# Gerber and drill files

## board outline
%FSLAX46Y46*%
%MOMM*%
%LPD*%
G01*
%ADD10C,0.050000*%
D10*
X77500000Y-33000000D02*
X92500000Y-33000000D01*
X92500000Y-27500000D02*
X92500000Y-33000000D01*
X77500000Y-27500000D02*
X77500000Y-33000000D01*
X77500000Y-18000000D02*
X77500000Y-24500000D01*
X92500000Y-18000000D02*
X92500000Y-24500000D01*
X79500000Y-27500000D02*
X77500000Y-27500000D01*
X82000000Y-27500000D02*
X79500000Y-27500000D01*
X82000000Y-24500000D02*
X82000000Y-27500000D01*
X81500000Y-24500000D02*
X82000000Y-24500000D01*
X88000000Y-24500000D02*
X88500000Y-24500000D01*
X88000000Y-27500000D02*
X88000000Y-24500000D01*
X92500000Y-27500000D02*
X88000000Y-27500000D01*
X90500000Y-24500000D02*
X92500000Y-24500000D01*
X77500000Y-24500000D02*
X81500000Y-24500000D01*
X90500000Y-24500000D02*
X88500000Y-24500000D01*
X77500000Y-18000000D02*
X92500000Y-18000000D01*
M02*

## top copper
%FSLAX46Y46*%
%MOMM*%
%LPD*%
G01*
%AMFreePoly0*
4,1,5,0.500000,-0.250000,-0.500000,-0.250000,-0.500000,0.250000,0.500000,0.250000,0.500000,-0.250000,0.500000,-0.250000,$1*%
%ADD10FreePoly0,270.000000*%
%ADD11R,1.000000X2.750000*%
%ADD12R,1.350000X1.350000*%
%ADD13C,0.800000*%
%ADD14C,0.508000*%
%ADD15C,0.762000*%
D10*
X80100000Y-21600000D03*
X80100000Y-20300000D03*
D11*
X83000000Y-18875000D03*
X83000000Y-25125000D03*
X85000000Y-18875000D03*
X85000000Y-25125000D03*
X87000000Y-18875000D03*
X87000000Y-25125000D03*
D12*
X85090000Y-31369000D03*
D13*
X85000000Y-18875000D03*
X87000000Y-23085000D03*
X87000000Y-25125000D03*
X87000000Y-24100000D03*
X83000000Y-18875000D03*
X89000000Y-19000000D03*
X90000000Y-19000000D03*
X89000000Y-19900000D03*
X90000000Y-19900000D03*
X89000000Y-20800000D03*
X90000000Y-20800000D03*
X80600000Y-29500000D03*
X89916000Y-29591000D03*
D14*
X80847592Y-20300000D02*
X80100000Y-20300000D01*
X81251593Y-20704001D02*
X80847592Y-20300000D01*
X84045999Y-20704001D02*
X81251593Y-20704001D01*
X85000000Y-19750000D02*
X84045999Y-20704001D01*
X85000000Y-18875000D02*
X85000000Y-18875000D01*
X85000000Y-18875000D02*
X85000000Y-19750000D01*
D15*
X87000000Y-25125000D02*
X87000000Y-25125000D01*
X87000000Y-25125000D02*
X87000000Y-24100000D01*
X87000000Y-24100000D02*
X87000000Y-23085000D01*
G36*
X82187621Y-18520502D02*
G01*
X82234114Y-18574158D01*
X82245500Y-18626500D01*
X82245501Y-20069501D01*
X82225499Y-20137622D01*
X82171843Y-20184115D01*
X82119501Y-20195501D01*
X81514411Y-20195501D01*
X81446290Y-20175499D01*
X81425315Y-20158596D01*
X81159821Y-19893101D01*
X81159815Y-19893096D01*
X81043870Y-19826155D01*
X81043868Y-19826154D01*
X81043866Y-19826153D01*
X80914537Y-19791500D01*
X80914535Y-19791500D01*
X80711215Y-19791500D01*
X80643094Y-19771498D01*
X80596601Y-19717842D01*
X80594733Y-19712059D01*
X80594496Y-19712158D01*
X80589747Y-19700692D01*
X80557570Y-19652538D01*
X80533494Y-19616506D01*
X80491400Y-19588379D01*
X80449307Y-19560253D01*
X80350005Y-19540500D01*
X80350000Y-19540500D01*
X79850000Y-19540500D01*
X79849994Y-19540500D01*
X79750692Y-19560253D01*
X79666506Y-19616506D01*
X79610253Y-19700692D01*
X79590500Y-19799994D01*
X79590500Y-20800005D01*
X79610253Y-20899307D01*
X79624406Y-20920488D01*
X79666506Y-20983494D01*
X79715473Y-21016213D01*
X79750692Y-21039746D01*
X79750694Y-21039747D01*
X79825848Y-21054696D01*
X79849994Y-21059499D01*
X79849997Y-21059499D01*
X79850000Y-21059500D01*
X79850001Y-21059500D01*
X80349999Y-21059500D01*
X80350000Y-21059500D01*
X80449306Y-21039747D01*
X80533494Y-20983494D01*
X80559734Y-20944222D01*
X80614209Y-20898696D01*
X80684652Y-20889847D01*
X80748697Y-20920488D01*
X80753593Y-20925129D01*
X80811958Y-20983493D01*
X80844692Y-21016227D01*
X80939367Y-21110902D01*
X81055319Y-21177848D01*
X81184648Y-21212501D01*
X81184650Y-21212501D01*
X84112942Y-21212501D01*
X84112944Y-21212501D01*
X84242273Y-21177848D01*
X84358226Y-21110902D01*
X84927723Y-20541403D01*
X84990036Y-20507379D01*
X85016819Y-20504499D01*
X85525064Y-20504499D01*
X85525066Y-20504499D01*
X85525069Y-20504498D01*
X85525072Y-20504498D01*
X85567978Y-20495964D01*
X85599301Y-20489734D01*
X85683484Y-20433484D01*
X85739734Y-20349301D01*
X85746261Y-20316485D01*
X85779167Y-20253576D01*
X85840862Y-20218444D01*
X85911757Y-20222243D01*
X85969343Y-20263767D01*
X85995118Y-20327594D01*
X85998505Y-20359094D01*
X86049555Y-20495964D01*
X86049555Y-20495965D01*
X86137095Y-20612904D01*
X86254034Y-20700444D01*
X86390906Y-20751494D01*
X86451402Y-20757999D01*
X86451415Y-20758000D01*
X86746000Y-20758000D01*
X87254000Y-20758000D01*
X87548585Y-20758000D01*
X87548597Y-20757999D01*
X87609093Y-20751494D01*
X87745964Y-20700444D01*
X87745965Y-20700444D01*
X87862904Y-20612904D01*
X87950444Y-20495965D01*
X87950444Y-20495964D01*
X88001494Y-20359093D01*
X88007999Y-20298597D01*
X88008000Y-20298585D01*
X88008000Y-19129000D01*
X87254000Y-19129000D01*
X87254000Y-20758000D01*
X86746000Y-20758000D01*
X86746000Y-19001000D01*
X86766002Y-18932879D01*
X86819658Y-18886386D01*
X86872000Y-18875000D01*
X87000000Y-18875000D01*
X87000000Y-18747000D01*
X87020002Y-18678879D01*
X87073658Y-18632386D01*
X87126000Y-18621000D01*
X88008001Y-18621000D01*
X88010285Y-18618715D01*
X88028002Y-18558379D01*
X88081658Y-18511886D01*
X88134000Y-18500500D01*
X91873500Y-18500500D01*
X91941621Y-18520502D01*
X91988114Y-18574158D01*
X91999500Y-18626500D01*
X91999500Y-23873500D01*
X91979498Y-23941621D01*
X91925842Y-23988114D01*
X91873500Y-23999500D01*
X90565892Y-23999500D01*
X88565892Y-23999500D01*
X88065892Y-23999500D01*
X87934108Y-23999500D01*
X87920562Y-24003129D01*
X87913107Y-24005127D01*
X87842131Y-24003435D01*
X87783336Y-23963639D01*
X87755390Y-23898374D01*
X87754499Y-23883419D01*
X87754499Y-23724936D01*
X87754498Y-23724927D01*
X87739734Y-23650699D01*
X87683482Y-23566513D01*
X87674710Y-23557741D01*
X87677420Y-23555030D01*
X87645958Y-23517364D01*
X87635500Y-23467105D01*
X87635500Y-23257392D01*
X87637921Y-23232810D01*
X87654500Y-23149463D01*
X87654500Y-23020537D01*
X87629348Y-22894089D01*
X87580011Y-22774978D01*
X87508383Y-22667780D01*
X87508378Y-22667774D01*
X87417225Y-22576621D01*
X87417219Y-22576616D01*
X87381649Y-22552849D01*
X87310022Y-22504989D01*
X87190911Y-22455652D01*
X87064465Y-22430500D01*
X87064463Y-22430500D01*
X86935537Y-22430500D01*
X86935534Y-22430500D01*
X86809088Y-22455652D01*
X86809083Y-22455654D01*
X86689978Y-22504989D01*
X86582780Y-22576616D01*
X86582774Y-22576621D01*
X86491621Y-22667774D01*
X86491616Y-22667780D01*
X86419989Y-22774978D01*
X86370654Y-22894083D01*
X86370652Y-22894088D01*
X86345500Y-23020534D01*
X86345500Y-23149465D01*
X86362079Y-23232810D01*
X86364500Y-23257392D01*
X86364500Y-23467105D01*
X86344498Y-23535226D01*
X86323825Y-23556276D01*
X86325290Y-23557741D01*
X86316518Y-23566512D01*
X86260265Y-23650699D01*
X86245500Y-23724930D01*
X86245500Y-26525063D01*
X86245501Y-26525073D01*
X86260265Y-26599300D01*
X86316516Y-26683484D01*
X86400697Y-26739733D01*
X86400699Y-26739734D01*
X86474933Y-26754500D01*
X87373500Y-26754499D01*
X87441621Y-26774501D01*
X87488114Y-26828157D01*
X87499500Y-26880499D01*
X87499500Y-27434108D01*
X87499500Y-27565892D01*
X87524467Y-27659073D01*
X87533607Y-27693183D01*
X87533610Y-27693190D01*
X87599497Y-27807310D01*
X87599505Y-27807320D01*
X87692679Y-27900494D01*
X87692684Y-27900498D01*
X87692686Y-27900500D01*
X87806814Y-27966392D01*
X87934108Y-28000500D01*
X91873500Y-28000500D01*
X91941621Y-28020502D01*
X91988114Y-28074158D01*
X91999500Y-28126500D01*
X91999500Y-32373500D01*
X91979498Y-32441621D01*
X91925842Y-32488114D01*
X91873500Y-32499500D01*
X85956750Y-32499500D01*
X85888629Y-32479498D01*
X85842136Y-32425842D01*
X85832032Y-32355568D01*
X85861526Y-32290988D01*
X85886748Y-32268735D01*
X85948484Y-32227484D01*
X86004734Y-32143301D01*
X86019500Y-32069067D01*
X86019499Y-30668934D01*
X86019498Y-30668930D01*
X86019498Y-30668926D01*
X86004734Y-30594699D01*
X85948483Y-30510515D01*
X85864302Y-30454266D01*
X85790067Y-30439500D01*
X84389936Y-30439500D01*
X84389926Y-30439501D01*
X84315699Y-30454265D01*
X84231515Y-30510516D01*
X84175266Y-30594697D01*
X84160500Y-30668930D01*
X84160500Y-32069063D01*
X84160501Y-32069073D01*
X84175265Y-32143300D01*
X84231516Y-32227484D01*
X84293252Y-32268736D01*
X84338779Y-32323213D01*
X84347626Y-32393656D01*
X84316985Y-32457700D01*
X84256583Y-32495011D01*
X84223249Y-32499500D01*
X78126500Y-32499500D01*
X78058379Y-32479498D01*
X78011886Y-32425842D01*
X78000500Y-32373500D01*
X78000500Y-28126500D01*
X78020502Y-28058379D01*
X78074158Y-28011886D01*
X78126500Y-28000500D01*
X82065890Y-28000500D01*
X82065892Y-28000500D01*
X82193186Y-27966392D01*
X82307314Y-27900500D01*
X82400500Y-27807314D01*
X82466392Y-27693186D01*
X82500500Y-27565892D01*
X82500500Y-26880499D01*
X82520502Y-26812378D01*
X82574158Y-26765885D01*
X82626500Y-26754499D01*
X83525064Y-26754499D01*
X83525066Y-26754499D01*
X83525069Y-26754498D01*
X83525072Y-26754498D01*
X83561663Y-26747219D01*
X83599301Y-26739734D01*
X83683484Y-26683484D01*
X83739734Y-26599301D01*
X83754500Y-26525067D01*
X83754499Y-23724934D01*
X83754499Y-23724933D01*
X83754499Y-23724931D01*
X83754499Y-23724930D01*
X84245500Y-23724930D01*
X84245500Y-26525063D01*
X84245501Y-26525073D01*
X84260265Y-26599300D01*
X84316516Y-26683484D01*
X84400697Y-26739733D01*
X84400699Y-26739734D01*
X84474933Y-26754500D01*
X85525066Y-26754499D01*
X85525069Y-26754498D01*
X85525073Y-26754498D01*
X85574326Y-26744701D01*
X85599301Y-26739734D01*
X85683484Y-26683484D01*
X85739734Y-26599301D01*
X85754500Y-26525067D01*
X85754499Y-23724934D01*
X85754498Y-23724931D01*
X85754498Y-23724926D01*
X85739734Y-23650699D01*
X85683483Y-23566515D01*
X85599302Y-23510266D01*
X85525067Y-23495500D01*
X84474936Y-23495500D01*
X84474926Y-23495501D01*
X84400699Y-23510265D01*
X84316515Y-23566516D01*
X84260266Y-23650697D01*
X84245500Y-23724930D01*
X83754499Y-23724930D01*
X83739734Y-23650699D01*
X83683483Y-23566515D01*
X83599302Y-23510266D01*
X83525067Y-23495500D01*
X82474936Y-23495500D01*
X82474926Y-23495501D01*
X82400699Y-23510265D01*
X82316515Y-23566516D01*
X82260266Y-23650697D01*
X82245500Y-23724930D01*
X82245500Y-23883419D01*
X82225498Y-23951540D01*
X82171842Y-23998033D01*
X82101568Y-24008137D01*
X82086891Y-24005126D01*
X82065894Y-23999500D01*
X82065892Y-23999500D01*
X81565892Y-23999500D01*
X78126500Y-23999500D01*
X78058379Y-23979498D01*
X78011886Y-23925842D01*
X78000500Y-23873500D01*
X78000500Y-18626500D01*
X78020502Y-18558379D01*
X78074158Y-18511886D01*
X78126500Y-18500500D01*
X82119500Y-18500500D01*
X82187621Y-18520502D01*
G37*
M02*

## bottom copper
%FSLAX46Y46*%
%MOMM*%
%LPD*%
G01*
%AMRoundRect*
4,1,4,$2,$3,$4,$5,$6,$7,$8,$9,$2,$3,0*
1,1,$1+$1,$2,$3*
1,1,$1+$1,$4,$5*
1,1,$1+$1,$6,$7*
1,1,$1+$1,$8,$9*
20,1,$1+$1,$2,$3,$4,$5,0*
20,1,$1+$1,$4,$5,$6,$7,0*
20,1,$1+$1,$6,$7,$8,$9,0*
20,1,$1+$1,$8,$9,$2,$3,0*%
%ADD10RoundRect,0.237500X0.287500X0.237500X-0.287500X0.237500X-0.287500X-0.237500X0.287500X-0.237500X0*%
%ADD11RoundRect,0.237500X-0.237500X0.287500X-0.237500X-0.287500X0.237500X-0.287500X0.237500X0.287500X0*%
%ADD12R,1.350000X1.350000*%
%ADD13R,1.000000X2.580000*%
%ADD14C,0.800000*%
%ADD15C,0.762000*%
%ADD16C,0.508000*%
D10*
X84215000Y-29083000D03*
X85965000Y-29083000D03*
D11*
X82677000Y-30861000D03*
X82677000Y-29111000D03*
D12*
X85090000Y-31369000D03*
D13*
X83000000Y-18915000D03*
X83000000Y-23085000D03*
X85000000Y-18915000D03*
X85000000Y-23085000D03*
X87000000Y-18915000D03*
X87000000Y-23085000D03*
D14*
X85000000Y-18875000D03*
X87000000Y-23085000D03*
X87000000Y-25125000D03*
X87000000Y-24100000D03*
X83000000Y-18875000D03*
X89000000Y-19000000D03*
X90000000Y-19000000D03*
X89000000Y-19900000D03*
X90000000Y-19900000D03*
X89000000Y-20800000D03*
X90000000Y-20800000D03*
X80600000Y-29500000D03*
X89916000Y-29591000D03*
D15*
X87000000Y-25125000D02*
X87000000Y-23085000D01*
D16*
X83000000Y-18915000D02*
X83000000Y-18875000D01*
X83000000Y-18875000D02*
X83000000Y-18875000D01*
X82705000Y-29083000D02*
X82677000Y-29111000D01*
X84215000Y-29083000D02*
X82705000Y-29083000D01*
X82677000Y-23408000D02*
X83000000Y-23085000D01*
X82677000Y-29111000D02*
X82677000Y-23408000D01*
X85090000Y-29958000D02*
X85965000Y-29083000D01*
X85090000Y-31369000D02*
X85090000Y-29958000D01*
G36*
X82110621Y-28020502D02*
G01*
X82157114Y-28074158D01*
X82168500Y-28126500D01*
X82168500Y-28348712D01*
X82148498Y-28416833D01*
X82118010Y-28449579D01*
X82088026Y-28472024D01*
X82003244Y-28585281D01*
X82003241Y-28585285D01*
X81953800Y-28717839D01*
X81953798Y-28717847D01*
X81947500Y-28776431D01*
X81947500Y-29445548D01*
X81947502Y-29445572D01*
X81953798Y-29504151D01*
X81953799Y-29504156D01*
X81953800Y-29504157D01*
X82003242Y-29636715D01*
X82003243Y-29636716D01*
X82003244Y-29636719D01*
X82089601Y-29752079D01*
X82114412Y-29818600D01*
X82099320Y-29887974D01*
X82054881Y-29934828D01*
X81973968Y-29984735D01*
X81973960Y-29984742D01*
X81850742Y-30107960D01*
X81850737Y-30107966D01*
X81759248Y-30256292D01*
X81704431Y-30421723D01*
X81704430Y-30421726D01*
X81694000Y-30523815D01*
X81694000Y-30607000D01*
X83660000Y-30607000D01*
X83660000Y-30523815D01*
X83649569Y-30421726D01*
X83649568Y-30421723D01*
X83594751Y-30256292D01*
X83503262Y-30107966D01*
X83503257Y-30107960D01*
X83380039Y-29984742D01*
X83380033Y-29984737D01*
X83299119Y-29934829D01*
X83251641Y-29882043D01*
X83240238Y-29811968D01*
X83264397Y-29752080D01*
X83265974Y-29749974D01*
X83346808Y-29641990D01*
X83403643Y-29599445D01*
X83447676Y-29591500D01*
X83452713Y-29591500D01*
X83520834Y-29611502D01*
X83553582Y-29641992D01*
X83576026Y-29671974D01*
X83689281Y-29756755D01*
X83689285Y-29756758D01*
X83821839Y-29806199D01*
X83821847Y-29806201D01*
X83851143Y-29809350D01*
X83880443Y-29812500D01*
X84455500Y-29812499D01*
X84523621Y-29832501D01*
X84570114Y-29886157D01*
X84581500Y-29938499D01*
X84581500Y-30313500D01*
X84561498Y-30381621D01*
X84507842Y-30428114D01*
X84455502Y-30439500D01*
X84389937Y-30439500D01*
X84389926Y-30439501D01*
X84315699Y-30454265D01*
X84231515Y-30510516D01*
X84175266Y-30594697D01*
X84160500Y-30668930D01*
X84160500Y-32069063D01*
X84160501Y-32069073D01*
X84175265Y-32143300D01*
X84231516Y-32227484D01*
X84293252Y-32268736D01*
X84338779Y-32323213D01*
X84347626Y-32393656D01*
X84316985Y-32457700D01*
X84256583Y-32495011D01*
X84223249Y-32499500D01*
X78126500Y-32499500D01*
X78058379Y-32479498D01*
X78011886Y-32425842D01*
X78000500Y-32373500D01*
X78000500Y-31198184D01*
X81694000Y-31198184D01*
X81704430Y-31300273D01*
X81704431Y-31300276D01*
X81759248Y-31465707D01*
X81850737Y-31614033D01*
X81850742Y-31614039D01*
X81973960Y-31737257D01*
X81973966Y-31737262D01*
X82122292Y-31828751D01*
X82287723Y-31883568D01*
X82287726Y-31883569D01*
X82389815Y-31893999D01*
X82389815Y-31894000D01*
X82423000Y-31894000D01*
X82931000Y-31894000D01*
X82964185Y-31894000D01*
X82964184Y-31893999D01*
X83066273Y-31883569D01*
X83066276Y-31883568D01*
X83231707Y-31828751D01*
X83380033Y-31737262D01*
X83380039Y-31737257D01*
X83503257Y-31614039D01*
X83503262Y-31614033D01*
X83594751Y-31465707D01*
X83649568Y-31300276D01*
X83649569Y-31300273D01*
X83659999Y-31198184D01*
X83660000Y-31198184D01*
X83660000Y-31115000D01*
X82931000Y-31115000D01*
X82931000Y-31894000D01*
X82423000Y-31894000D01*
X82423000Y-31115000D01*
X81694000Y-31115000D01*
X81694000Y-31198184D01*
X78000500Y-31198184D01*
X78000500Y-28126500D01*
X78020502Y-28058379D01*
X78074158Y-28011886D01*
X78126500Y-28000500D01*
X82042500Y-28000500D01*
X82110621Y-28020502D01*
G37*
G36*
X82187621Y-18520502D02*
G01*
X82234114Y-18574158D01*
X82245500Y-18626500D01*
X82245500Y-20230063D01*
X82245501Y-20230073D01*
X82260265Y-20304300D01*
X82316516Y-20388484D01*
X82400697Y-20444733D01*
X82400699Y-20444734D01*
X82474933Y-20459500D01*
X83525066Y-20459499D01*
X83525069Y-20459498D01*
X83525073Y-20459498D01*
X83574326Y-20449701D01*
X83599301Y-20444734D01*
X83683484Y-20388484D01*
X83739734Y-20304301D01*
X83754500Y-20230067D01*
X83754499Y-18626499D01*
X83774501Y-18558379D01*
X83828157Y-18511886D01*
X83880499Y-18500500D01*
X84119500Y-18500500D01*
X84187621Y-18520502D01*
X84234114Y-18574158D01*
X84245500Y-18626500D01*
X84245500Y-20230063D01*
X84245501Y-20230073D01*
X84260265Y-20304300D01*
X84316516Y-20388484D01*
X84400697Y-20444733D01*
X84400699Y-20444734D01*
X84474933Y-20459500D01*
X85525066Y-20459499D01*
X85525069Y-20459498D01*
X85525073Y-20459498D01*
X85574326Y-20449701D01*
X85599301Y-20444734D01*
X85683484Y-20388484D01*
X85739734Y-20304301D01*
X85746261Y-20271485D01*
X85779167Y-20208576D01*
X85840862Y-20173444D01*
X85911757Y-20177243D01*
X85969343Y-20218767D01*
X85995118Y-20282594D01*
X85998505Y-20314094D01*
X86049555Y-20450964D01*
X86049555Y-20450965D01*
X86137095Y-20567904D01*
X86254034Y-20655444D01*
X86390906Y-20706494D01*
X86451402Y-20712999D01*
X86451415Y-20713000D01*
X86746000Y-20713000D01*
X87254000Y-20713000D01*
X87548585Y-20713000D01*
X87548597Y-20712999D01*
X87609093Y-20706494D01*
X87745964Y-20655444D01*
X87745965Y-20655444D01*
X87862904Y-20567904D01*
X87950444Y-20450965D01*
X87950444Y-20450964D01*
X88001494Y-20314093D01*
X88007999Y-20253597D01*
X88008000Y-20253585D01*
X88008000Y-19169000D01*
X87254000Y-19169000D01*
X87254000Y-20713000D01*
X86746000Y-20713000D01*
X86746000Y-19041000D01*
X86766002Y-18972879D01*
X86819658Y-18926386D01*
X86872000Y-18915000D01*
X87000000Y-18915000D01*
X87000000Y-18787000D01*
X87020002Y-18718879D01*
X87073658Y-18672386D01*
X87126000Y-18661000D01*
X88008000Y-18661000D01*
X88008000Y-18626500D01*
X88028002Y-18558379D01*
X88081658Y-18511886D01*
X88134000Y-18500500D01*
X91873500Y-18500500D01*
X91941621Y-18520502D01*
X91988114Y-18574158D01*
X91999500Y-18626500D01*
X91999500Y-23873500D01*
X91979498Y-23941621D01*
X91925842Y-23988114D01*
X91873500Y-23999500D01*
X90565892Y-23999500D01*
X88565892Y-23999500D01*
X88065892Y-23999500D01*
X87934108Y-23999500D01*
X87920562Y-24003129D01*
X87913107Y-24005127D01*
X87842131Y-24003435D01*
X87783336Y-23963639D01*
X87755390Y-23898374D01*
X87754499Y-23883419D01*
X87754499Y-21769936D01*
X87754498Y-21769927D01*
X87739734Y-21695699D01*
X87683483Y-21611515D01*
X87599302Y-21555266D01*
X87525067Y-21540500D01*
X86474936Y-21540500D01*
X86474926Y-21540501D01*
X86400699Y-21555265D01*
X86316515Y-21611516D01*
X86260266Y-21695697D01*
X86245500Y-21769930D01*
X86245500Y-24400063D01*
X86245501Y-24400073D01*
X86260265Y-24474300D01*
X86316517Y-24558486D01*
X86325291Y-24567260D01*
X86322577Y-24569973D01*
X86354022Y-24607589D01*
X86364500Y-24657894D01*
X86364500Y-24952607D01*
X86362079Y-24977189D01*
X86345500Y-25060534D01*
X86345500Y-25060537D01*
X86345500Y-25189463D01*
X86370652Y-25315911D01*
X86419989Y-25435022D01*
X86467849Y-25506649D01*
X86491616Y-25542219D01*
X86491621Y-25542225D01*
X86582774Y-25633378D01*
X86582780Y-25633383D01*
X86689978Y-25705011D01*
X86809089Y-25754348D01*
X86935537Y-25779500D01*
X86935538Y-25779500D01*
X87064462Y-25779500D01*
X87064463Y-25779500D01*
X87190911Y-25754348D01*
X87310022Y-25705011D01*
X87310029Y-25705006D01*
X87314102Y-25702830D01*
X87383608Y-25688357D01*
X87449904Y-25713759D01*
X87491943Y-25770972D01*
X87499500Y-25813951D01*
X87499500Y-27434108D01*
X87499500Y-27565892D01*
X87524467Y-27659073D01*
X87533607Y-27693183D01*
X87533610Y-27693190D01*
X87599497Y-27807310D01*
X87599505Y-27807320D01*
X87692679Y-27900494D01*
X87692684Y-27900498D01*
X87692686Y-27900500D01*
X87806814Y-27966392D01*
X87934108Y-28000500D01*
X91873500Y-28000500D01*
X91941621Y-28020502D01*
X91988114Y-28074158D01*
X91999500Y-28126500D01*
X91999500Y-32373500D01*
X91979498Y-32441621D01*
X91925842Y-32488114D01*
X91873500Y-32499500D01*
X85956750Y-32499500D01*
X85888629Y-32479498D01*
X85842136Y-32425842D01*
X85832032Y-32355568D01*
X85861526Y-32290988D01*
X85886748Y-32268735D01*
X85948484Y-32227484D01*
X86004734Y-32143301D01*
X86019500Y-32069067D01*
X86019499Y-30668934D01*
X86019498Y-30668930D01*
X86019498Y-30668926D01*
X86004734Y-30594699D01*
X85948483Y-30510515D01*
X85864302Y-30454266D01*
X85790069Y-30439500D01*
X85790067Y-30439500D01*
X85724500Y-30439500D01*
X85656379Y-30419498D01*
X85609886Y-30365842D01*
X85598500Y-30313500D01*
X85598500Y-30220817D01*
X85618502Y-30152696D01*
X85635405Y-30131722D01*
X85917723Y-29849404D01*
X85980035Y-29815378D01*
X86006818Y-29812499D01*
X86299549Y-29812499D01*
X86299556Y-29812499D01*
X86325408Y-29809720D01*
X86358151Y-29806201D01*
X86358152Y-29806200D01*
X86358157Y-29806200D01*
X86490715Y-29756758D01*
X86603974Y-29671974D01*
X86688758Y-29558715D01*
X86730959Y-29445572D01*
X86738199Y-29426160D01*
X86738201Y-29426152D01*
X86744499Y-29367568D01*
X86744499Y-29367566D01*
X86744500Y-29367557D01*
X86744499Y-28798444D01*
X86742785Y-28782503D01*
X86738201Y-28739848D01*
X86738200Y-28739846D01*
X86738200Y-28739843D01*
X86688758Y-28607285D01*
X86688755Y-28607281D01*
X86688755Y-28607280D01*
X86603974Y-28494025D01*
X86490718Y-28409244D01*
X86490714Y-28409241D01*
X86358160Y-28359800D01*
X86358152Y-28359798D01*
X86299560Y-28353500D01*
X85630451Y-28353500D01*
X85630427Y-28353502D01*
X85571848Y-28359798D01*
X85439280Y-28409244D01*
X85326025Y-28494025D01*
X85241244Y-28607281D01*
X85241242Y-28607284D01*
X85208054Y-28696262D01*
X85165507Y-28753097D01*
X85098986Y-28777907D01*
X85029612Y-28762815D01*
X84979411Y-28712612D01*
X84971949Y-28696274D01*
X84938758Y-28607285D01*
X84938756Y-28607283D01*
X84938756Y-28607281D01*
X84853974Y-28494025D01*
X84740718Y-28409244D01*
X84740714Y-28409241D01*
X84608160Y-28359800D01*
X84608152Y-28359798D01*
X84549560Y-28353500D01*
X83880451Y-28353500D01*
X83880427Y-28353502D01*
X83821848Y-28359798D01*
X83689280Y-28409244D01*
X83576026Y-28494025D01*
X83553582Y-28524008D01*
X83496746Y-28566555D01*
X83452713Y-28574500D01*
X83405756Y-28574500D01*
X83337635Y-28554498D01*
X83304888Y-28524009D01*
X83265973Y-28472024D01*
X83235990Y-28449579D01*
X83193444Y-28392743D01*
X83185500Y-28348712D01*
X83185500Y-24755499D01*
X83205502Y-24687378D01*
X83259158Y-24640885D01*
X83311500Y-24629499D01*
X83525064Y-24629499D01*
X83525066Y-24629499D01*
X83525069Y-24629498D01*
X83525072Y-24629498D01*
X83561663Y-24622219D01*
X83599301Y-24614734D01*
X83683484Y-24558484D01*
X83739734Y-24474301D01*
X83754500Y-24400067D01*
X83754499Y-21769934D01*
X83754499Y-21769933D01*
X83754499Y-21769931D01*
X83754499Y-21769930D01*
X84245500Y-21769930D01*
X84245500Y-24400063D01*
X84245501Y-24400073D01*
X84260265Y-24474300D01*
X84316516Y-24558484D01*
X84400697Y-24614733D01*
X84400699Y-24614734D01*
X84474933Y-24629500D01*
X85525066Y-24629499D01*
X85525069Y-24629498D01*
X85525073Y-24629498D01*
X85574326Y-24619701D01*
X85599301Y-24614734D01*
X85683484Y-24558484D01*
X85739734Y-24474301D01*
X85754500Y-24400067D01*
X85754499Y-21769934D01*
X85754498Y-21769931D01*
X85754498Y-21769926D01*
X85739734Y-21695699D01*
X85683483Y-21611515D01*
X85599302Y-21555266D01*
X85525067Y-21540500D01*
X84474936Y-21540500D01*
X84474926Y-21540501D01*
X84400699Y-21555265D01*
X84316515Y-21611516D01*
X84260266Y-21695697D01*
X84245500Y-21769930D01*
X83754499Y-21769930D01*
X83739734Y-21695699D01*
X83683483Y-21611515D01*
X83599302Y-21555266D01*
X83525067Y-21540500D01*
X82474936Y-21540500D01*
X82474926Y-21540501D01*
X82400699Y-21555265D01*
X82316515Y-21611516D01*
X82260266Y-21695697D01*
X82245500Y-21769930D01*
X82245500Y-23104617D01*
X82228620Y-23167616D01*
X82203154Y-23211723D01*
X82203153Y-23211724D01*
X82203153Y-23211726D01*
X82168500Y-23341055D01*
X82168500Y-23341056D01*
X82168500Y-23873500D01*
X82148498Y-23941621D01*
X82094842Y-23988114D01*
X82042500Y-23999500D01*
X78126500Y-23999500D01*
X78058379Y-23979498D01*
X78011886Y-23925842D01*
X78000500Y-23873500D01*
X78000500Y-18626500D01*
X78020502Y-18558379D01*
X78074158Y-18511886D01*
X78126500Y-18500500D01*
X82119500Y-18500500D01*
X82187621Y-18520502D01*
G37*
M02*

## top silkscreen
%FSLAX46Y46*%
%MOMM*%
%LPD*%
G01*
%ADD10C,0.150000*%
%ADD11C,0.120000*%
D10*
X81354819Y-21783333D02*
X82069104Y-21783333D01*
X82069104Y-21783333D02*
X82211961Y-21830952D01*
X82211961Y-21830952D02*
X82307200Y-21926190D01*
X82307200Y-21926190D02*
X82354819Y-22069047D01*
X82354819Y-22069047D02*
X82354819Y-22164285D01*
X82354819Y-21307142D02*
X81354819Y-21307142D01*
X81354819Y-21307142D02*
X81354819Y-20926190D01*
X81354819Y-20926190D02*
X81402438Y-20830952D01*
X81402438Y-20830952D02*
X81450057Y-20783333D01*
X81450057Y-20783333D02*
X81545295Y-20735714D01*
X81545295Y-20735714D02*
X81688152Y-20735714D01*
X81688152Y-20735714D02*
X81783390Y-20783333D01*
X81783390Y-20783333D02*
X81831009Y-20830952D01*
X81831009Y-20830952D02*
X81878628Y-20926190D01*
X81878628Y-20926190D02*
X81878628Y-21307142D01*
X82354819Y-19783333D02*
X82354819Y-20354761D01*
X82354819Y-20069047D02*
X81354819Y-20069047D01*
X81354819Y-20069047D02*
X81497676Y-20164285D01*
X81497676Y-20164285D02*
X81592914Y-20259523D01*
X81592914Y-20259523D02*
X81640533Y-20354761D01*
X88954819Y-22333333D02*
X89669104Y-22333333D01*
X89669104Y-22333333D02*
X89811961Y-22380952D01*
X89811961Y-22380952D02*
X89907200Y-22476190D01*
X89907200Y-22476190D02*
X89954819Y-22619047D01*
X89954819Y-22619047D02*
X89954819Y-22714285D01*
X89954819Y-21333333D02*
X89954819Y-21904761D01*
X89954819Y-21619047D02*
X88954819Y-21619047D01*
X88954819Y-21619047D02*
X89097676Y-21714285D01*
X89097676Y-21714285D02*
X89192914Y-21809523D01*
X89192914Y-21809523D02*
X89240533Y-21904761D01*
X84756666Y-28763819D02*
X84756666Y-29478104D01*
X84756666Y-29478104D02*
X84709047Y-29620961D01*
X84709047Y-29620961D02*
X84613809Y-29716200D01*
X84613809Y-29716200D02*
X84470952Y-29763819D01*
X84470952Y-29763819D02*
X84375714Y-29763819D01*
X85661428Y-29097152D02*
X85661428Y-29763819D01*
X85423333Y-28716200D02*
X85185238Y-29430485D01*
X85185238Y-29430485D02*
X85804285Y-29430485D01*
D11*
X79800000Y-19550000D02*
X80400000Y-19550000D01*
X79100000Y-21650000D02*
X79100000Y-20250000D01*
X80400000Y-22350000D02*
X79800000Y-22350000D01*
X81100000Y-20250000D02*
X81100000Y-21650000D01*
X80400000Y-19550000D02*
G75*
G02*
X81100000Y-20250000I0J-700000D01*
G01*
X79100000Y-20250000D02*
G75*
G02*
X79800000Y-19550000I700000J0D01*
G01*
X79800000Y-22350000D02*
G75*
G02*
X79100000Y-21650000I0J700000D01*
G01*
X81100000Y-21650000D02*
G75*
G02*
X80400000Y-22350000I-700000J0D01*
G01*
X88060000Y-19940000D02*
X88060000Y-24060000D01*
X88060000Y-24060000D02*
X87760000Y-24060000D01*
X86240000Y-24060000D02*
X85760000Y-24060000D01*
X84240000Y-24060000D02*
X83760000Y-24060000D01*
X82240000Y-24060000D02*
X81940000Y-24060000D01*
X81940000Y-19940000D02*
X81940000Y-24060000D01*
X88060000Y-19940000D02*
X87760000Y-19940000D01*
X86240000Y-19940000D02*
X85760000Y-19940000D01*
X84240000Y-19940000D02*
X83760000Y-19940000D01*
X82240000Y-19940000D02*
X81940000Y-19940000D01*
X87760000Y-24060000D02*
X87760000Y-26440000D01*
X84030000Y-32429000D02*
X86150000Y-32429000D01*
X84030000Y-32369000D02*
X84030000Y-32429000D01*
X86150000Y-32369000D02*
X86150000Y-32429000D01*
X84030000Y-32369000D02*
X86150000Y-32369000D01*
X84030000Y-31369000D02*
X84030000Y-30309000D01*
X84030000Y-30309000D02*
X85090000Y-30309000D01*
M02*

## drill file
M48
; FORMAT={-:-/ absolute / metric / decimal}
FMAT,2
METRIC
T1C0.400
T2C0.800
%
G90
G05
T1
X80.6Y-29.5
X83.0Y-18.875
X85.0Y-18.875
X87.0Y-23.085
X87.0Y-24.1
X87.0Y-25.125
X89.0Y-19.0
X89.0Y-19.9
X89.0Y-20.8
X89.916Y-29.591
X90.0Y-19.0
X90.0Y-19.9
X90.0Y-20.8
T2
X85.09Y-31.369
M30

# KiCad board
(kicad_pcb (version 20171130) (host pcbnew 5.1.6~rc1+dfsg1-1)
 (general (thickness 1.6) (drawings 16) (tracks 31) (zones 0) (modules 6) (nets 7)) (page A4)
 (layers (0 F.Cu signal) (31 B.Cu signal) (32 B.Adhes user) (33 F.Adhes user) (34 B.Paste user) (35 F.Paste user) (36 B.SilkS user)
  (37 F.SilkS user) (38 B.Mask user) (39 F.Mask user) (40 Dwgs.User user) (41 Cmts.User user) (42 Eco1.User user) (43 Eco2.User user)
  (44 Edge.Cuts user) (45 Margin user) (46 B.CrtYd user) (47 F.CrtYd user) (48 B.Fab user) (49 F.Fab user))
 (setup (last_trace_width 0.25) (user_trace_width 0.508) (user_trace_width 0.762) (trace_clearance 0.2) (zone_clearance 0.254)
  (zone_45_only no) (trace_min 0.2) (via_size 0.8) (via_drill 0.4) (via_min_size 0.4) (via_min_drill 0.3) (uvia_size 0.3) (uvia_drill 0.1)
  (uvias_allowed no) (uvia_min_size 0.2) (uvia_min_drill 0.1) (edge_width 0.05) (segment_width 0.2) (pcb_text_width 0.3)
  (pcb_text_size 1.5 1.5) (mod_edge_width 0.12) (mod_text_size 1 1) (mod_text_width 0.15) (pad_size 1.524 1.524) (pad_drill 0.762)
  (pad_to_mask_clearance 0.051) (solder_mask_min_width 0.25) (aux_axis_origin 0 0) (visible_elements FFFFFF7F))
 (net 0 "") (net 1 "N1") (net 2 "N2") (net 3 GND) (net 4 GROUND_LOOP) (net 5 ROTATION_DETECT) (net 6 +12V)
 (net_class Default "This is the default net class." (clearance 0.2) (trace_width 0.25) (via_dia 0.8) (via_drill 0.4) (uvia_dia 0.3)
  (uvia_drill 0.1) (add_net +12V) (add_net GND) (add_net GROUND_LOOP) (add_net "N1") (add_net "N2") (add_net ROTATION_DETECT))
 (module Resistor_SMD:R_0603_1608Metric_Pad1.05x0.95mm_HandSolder (layer B.Cu) (at 85.09 29.083 180)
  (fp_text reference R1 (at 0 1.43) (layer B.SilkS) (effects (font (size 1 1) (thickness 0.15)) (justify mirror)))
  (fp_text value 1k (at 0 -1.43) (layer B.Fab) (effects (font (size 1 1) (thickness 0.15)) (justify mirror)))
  (pad 2 smd roundrect (at 0.875 0 180) (size 1.05 0.95) (layers B.Cu B.Paste B.Mask) (roundrect_rratio 0.25) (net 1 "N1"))
  (pad 1 smd roundrect (at -0.875 0 180) (size 1.05 0.95) (layers B.Cu B.Paste B.Mask) (roundrect_rratio 0.25) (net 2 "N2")))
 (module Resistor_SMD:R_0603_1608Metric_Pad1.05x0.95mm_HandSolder (layer B.Cu) (at 82.677 29.986 270)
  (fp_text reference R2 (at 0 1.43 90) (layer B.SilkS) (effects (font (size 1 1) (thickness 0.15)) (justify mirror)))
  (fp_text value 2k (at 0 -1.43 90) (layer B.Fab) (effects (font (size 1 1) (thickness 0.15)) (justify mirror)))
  (pad 2 smd roundrect (at 0.875 0 270) (size 1.05 0.95) (layers B.Cu B.Paste B.Mask) (roundrect_rratio 0.25) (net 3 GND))
  (pad 1 smd roundrect (at -0.875 0 270) (size 1.05 0.95) (layers B.Cu B.Paste B.Mask) (roundrect_rratio 0.25) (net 1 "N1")))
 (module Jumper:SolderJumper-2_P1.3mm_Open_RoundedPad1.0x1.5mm (layer F.Cu) (at 80.1 20.95 270)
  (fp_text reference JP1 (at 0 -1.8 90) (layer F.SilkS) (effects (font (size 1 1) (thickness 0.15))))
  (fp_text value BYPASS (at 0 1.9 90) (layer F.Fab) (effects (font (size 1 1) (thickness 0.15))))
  (fp_line (start -1.4 0.3) (end -1.4 -0.3) (layer F.SilkS) (width 0.12))
  (fp_line (start 0.7 1) (end -0.7 1) (layer F.SilkS) (width 0.12))
  (fp_line (start 1.4 -0.3) (end 1.4 0.3) (layer F.SilkS) (width 0.12))
  (fp_line (start -0.7 -1) (end 0.7 -1) (layer F.SilkS) (width 0.12))
  (fp_arc (start -0.7 -0.3) (end -0.7 -1) (angle -90) (layer F.SilkS) (width 0.12))
  (fp_arc (start -0.7 0.3) (end -1.4 0.3) (angle -90) (layer F.SilkS) (width 0.12))
  (fp_arc (start 0.7 0.3) (end 0.7 1) (angle -90) (layer F.SilkS) (width 0.12))
  (fp_arc (start 0.7 -0.3) (end 1.4 -0.3) (angle -90) (layer F.SilkS) (width 0.12))
  (pad 2 smd custom (at 0.65 0 270) (size 1 0.5) (layers F.Cu F.Mask) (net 3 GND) (zone_connect 2)
   (options (clearance outline) (anchor rect)) (primitives))
  (pad 1 smd custom (at -0.65 0 270) (size 1 0.5) (layers F.Cu F.Mask) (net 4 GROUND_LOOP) (zone_connect 2)
   (options (clearance outline) (anchor rect)) (primitives)))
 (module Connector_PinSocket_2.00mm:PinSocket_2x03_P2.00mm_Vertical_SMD (layer F.Cu) (at 85 22 270)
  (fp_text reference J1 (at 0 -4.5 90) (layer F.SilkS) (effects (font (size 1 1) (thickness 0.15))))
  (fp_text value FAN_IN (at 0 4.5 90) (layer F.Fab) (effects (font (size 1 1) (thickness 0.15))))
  (fp_line (start -2.06 -3.06) (end 2.06 -3.06) (layer F.SilkS) (width 0.12))
  (fp_line (start 2.06 -3.06) (end 2.06 -2.76) (layer F.SilkS) (width 0.12))
  (fp_line (start 2.06 -1.24) (end 2.06 -0.76) (layer F.SilkS) (width 0.12))
  (fp_line (start 2.06 0.76) (end 2.06 1.24) (layer F.SilkS) (width 0.12))
  (fp_line (start 2.06 2.76) (end 2.06 3.06) (layer F.SilkS) (width 0.12))
  (fp_line (start -2.06 3.06) (end 2.06 3.06) (layer F.SilkS) (width 0.12))
  (fp_line (start -2.06 -3.06) (end -2.06 -2.76) (layer F.SilkS) (width 0.12))
  (fp_line (start -2.06 -1.24) (end -2.06 -0.76) (layer F.SilkS) (width 0.12))
  (fp_line (start -2.06 0.76) (end -2.06 1.24) (layer F.SilkS) (width 0.12))
  (fp_line (start -2.06 2.76) (end -2.06 3.06) (layer F.SilkS) (width 0.12))
  (fp_line (start 2.06 -2.76) (end 4.44 -2.76) (layer F.SilkS) (width 0.12))
  (pad 6 smd rect (at -3.125 2 270) (size 2.75 1) (layers F.Cu F.Paste F.Mask) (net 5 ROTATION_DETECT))
  (pad 5 smd rect (at 3.125 2 270) (size 2.75 1) (layers F.Cu F.Paste F.Mask))
  (pad 4 smd rect (at -3.125 0 270) (size 2.75 1) (layers F.Cu F.Paste F.Mask) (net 4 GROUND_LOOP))
  (pad 3 smd rect (at 3.125 0 270) (size 2.75 1) (layers F.Cu F.Paste F.Mask))
  (pad 2 smd rect (at -3.125 -2 270) (size 2.75 1) (layers F.Cu F.Paste F.Mask) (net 3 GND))
  (pad 1 smd rect (at 3.125 -2 270) (size 2.75 1) (layers F.Cu F.Paste F.Mask) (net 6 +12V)))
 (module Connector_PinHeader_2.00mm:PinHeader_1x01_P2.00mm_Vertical (layer F.Cu) (at 85.09 31.369)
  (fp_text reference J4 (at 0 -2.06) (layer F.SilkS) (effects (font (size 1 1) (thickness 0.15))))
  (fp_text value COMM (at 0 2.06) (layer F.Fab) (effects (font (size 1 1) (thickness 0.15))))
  (fp_line (start -1.06 1.06) (end 1.06 1.06) (layer F.SilkS) (width 0.12))
  (fp_line (start -1.06 1) (end -1.06 1.06) (layer F.SilkS) (width 0.12))
  (fp_line (start 1.06 1) (end 1.06 1.06) (layer F.SilkS) (width 0.12))
  (fp_line (start -1.06 1) (end 1.06 1) (layer F.SilkS) (width 0.12))
  (fp_line (start -1.06 0) (end -1.06 -1.06) (layer F.SilkS) (width 0.12))
  (fp_line (start -1.06 -1.06) (end 0 -1.06) (layer F.SilkS) (width 0.12))
  (pad 1 thru_hole rect (at 0 0) (size 1.35 1.35) (drill 0.8) (layers *.Cu *.Mask) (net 2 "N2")))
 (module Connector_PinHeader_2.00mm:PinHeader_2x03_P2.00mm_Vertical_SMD (layer B.Cu) (at 85 21 90)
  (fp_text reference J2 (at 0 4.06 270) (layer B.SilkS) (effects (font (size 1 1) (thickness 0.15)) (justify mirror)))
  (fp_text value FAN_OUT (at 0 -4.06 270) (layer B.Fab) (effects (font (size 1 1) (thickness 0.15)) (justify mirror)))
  (pad 6 smd rect (at 2.085 -2 90) (size 2.58 1) (layers B.Cu B.Paste B.Mask) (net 5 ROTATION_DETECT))
  (pad 5 smd rect (at -2.085 -2 90) (size 2.58 1) (layers B.Cu B.Paste B.Mask) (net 1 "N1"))
  (pad 4 smd rect (at 2.085 0 90) (size 2.58 1) (layers B.Cu B.Paste B.Mask) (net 4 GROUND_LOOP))
  (pad 3 smd rect (at -2.085 0 90) (size 2.58 1) (layers B.Cu B.Paste B.Mask))
  (pad 2 smd rect (at 2.085 2 90) (size 2.58 1) (layers B.Cu B.Paste B.Mask) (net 3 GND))
  (pad 1 smd rect (at -2.085 2 90) (size 2.58 1) (layers B.Cu B.Paste B.Mask) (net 6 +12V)))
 (gr_line (start 77.5 33) (end 92.5 33) (layer Edge.Cuts) (width 0.05))
 (gr_line (start 92.5 27.5) (end 92.5 33) (layer Edge.Cuts) (width 0.05))
 (gr_line (start 77.5 27.5) (end 77.5 33) (layer Edge.Cuts) (width 0.05))
 (gr_line (start 77.5 18) (end 77.5 24.5) (layer Edge.Cuts) (width 0.05))
 (gr_line (start 92.5 18) (end 92.5 24.5) (layer Edge.Cuts) (width 0.05))
 (gr_line (start 79.5 27.5) (end 77.5 27.5) (layer Edge.Cuts) (width 0.05))
 (gr_line (start 82 27.5) (end 79.5 27.5) (layer Edge.Cuts) (width 0.05))
 (gr_line (start 82 24.5) (end 82 27.5) (layer Edge.Cuts) (width 0.05))
 (gr_line (start 81.5 24.5) (end 82 24.5) (layer Edge.Cuts) (width 0.05))
 (gr_line (start 88 24.5) (end 88.5 24.5) (layer Edge.Cuts) (width 0.05))
 (gr_line (start 88 27.5) (end 88 24.5) (layer Edge.Cuts) (width 0.05))
 (gr_line (start 92.5 27.5) (end 88 27.5) (layer Edge.Cuts) (width 0.05))
 (gr_line (start 90.5 24.5) (end 92.5 24.5) (layer Edge.Cuts) (width 0.05))
 (gr_line (start 77.5 24.5) (end 81.5 24.5) (layer Edge.Cuts) (width 0.05))
 (gr_line (start 90.5 24.5) (end 88.5 24.5) (layer Edge.Cuts) (width 0.05))
 (gr_line (start 77.5 18) (end 92.5 18) (layer Edge.Cuts) (width 0.05))
 (segment (start 80.847592 20.3) (end 80.1 20.3) (width 0.508) (layer F.Cu) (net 4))
 (segment (start 81.251593 20.704001) (end 80.847592 20.3) (width 0.508) (layer F.Cu) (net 4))
 (segment (start 84.045999 20.704001) (end 81.251593 20.704001) (width 0.508) (layer F.Cu) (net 4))
 (segment (start 85 19.75) (end 84.045999 20.704001) (width 0.508) (layer F.Cu) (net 4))
 (segment (start 85 18.875) (end 85 18.875) (width 0.508) (layer F.Cu) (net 4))
 (segment (start 85 18.875) (end 85 19.75) (width 0.508) (layer F.Cu) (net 4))
 (via (at 85 18.875) (size 0.8) (drill 0.4) (layers F.Cu B.Cu) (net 4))
 (via (at 87 23.085) (size 0.8) (drill 0.4) (layers F.Cu B.Cu) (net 6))
 (segment (start 87 25.125) (end 87 25.125) (width 0.762) (layer F.Cu) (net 6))
 (segment (start 87 25.125) (end 87 24.1) (width 0.762) (layer F.Cu) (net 6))
 (via (at 87 25.125) (size 0.8) (drill 0.4) (layers F.Cu B.Cu) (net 6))
 (segment (start 87 24.1) (end 87 23.085) (width 0.762) (layer F.Cu) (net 6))
 (via (at 87 24.1) (size 0.8) (drill 0.4) (layers F.Cu B.Cu) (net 6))
 (segment (start 87 25.125) (end 87 23.085) (width 0.762) (layer B.Cu) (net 6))
 (segment (start 83 18.915) (end 83 18.875) (width 0.508) (layer B.Cu) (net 5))
 (segment (start 83 18.875) (end 83 18.875) (width 0.508) (layer B.Cu) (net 5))
 (via (at 83 18.875) (size 0.8) (drill 0.4) (layers F.Cu B.Cu) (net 5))
 (segment (start 82.705 29.083) (end 82.677 29.111) (width 0.508) (layer B.Cu) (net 1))
 (segment (start 84.215 29.083) (end 82.705 29.083) (width 0.508) (layer B.Cu) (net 1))
 (segment (start 82.677 23.408) (end 83 23.085) (width 0.508) (layer B.Cu) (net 1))
 (segment (start 82.677 29.111) (end 82.677 23.408) (width 0.508) (layer B.Cu) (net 1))
 (via (at 89 19) (size 0.8) (drill 0.4) (layers F.Cu B.Cu) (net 3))
 (via (at 90 19) (size 0.8) (drill 0.4) (layers F.Cu B.Cu) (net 3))
 (via (at 89 19.9) (size 0.8) (drill 0.4) (layers F.Cu B.Cu) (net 3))
 (via (at 90 19.9) (size 0.8) (drill 0.4) (layers F.Cu B.Cu) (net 3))
 (via (at 89 20.8) (size 0.8) (drill 0.4) (layers F.Cu B.Cu) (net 3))
 (via (at 90 20.8) (size 0.8) (drill 0.4) (layers F.Cu B.Cu) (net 3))
 (via (at 80.6 29.5) (size 0.8) (drill 0.4) (layers F.Cu B.Cu) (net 3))
 (via (at 89.916 29.591) (size 0.8) (drill 0.4) (layers F.Cu B.Cu) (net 3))
 (segment (start 85.09 29.958) (end 85.965 29.083) (width 0.508) (layer B.Cu) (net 2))
 (segment (start 85.09 31.369) (end 85.09 29.958) (width 0.508) (layer B.Cu) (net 2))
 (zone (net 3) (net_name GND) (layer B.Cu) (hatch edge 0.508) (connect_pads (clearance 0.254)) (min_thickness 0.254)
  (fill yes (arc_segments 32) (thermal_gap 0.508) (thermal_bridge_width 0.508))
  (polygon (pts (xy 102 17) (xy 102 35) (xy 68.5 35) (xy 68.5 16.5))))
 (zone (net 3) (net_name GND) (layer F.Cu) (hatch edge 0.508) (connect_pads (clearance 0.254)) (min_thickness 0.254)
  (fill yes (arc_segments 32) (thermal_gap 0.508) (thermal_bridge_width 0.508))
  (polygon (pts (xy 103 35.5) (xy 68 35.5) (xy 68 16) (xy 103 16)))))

